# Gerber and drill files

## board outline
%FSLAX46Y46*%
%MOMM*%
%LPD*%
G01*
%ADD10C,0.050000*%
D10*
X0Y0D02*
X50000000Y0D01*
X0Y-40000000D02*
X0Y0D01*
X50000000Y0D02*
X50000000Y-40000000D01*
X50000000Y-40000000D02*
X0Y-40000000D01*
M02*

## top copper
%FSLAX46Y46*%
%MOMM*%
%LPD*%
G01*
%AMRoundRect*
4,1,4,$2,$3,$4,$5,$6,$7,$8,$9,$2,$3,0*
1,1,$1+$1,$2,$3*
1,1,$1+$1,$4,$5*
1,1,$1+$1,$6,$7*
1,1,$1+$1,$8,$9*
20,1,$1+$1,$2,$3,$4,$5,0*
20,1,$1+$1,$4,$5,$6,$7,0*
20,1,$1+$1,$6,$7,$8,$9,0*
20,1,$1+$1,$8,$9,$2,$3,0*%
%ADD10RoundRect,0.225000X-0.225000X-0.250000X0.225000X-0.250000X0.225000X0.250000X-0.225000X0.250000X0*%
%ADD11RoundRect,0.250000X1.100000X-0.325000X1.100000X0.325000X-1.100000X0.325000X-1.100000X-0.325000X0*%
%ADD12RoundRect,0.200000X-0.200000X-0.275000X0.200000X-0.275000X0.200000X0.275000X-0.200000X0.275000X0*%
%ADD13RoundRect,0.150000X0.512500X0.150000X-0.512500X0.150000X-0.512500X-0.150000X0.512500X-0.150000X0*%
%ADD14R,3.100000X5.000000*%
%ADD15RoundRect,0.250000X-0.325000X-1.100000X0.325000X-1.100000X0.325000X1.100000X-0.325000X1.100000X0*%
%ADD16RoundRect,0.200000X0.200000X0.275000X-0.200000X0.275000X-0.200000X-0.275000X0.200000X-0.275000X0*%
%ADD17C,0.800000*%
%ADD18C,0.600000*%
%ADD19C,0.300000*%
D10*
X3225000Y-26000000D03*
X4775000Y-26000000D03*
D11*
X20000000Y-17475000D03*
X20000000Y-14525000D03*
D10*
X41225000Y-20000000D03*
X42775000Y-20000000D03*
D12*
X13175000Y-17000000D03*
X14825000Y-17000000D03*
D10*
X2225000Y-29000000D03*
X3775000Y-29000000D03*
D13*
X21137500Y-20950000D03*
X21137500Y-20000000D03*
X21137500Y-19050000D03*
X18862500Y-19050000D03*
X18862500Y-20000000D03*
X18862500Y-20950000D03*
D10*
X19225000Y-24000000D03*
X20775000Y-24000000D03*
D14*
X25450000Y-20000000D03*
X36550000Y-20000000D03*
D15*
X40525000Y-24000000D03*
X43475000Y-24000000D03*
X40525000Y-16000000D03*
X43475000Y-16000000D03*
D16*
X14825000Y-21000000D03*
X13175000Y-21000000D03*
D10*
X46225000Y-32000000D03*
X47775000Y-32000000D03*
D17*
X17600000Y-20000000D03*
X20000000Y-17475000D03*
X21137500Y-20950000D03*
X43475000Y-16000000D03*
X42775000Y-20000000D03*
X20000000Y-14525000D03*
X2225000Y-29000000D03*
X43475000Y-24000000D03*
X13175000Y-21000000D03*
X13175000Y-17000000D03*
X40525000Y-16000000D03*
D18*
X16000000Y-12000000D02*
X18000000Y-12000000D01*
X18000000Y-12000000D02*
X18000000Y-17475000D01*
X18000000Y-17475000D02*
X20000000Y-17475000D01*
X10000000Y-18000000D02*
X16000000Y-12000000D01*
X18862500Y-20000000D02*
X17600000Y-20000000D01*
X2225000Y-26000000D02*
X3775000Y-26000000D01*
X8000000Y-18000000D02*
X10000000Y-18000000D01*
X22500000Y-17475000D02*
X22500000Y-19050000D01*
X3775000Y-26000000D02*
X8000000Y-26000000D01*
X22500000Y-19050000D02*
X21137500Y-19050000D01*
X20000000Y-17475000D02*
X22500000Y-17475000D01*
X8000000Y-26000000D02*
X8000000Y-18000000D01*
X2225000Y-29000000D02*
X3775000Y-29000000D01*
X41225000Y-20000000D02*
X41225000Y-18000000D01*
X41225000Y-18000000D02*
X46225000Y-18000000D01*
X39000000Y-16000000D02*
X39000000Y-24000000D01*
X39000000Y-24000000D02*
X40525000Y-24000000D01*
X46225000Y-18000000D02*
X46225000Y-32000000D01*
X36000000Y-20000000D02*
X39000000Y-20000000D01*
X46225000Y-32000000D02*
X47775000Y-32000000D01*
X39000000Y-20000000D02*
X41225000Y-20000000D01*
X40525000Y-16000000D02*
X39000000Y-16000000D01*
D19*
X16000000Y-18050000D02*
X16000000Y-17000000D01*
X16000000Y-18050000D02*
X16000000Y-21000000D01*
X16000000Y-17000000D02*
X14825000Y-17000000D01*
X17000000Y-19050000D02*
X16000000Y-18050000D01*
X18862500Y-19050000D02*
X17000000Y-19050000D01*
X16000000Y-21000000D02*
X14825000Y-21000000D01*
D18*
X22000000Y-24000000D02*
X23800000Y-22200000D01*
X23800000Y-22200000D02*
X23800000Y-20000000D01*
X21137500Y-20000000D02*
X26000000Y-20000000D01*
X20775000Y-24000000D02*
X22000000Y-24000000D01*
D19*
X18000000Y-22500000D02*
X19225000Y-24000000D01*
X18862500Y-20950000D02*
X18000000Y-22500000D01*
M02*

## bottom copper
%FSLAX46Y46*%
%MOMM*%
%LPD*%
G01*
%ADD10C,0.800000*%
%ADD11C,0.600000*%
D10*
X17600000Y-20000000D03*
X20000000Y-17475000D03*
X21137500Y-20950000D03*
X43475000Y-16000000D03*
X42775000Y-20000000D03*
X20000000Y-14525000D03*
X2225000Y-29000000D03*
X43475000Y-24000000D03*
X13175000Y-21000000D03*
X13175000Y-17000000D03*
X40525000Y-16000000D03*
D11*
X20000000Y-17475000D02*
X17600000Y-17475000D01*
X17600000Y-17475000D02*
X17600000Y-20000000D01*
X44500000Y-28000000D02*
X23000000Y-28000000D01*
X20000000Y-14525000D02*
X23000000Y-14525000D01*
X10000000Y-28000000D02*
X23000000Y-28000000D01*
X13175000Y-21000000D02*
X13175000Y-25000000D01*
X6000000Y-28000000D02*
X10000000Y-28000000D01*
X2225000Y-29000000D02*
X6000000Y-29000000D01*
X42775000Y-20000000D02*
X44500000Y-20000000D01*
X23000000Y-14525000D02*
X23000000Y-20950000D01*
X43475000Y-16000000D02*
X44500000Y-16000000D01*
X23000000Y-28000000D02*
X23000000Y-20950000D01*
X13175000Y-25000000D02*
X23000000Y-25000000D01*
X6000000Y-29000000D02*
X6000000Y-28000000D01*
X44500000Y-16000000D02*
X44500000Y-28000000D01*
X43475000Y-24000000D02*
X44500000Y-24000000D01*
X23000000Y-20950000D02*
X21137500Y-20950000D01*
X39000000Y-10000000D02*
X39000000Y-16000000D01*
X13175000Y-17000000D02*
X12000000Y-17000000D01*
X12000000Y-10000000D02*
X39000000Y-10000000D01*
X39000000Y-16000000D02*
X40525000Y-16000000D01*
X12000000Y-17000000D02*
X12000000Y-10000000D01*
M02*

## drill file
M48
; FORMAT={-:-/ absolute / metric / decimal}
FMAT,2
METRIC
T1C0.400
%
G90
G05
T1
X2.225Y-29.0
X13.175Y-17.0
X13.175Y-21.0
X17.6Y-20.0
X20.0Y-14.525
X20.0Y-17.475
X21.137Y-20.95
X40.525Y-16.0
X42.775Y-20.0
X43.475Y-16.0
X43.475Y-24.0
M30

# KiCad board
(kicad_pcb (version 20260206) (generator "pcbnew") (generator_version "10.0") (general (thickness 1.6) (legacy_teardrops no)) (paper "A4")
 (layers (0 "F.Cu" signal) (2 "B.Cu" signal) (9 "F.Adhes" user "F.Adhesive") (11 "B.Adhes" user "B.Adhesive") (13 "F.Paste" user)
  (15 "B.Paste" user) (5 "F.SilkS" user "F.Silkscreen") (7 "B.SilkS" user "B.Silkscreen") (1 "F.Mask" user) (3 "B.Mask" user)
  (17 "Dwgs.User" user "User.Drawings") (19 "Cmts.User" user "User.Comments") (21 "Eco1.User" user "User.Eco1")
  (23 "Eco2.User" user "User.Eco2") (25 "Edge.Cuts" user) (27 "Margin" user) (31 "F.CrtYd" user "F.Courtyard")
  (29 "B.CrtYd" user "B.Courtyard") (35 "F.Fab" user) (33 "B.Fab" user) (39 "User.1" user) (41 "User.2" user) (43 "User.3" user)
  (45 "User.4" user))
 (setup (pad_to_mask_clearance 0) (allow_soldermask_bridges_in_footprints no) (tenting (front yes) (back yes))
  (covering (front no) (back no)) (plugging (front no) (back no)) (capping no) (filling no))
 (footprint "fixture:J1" (layer "F.Cu") (at 4 26)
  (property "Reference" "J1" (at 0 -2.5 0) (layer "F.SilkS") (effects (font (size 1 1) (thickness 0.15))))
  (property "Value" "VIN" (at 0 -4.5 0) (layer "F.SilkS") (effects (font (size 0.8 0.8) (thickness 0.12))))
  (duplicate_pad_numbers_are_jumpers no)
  (pad "1" smd roundrect (at -0.775 0) (size 0.9 0.95) (layers "F.Cu" "F.Mask" "F.Paste") (roundrect_rratio 0.25) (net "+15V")
   (thermal_bridge_angle 45))
  (pad "2" smd roundrect (at 0.775 0) (size 0.9 0.95) (layers "F.Cu" "F.Mask" "F.Paste") (roundrect_rratio 0.25) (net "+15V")
   (thermal_bridge_angle 45)))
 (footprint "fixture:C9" (layer "F.Cu") (at 20 16 90)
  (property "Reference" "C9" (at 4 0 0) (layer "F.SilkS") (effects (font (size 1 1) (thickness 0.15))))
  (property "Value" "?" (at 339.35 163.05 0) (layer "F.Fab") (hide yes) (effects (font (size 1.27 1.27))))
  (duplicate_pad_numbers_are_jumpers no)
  (pad "1" smd roundrect (at -1.475 0 90) (size 1.15 2.7) (layers "F.Cu" "F.Mask" "F.Paste") (roundrect_rratio 0.217391) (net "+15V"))
  (pad "2" smd roundrect (at 1.475 0 90) (size 1.15 2.7) (layers "F.Cu" "F.Mask" "F.Paste") (roundrect_rratio 0.217391) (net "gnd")))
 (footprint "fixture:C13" (layer "F.Cu") (at 42 20)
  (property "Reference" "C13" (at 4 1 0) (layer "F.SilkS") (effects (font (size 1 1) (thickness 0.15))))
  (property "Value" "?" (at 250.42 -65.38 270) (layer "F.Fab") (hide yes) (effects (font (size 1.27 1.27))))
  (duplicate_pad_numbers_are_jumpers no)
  (pad "1" smd roundrect (at -0.775 0) (size 0.9 0.95) (layers "F.Cu" "F.Mask" "F.Paste") (roundrect_rratio 0.25) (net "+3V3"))
  (pad "2" smd roundrect (at 0.775 0) (size 0.9 0.95) (layers "F.Cu" "F.Mask" "F.Paste") (roundrect_rratio 0.25) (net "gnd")))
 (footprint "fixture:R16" (layer "F.Cu") (at 14 17)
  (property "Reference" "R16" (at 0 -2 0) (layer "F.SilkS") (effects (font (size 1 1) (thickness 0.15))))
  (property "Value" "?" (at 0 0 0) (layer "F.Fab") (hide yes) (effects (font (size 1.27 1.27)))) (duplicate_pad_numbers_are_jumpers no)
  (pad "1" smd roundrect (at -0.825 0) (size 0.8 0.95) (layers "F.Cu" "F.Mask" "F.Paste") (roundrect_rratio 0.25) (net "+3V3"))
  (pad "2" smd roundrect (at 0.825 0) (size 0.8 0.95) (layers "F.Cu" "F.Mask" "F.Paste") (roundrect_rratio 0.25) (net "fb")))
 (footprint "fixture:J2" (layer "F.Cu") (at 3 29)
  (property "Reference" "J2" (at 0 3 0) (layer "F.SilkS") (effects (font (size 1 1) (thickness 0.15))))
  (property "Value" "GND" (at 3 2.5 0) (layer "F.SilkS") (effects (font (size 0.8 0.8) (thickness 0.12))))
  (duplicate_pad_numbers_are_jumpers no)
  (pad "1" smd roundrect (at -0.775 0) (size 0.9 0.95) (layers "F.Cu" "F.Mask" "F.Paste") (roundrect_rratio 0.25) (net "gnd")
   (thermal_bridge_angle 45))
  (pad "2" smd roundrect (at 0.775 0) (size 0.9 0.95) (layers "F.Cu" "F.Mask" "F.Paste") (roundrect_rratio 0.25) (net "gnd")
   (thermal_bridge_angle 45)))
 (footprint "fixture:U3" (layer "F.Cu") (at 20 20 180)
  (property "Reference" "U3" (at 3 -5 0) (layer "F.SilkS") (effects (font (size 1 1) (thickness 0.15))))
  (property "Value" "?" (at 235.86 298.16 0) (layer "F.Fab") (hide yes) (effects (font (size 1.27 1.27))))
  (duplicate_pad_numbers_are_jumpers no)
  (pad "1" smd roundrect (at -1.1375 -0.95 180) (size 1.325 0.6) (layers "F.Cu" "F.Mask" "F.Paste") (roundrect_rratio 0.25) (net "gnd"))
  (pad "2" smd roundrect (at -1.1375 0 180) (size 1.325 0.6) (layers "F.Cu" "F.Mask" "F.Paste") (roundrect_rratio 0.25) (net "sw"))
  (pad "3" smd roundrect (at -1.1375 0.95 180) (size 1.325 0.6) (layers "F.Cu" "F.Mask" "F.Paste") (roundrect_rratio 0.25) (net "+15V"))
  (pad "4" smd roundrect (at 1.1375 0.95 180) (size 1.325 0.6) (layers "F.Cu" "F.Mask" "F.Paste") (roundrect_rratio 0.25) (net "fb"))
  (pad "5" smd roundrect (at 1.1375 0 180) (size 1.325 0.6) (layers "F.Cu" "F.Mask" "F.Paste") (roundrect_rratio 0.25) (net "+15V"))
  (pad "6" smd roundrect (at 1.1375 -0.95 180) (size 1.325 0.6) (layers "F.Cu" "F.Mask" "F.Paste") (roundrect_rratio 0.25) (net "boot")))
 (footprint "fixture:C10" (layer "F.Cu") (at 20 24)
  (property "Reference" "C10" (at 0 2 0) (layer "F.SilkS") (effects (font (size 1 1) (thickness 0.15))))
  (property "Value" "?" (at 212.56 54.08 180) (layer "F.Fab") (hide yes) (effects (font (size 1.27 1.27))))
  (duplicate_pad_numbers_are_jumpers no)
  (pad "1" smd roundrect (at -0.775 0) (size 0.9 0.95) (layers "F.Cu" "F.Mask" "F.Paste") (roundrect_rratio 0.25) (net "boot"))
  (pad "2" smd roundrect (at 0.775 0) (size 0.9 0.95) (layers "F.Cu" "F.Mask" "F.Paste") (roundrect_rratio 0.25) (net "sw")))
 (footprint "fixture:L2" (layer "F.Cu") (at 31 20)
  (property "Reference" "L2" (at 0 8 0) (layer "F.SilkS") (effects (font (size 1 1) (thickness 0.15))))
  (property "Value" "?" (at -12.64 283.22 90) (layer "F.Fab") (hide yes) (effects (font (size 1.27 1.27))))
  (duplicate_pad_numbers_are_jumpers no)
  (pad "1" smd rect (at -5.55 0) (size 3.1 5) (layers "F.Cu" "F.Mask" "F.Paste") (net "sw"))
  (pad "2" smd rect (at 5.55 0) (size 3.1 5) (layers "F.Cu" "F.Mask" "F.Paste") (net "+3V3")))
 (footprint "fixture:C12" (layer "F.Cu") (at 42 24)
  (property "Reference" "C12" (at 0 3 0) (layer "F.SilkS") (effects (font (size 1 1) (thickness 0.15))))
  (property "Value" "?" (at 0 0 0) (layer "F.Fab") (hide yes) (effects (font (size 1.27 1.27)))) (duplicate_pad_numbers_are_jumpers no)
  (pad "1" smd roundrect (at -1.475 0) (size 1.15 2.7) (layers "F.Cu" "F.Mask" "F.Paste") (roundrect_rratio 0.217391) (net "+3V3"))
  (pad "2" smd roundrect (at 1.475 0) (size 1.15 2.7) (layers "F.Cu" "F.Mask" "F.Paste") (roundrect_rratio 0.217391) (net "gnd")))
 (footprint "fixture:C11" (layer "F.Cu") (at 42 16)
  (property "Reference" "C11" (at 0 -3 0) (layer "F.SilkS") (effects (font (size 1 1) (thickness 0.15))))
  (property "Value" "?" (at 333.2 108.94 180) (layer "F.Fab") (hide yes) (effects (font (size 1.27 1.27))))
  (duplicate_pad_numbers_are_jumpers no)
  (pad "1" smd roundrect (at -1.475 0) (size 1.15 2.7) (layers "F.Cu" "F.Mask" "F.Paste") (roundrect_rratio 0.217391) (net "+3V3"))
  (pad "2" smd roundrect (at 1.475 0) (size 1.15 2.7) (layers "F.Cu" "F.Mask" "F.Paste") (roundrect_rratio 0.217391) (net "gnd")))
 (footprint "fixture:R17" (layer "F.Cu") (at 14 21 180)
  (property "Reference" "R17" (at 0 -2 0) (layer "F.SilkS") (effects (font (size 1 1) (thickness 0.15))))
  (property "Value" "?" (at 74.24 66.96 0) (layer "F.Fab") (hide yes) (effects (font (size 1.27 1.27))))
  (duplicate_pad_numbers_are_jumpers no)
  (pad "1" smd roundrect (at -0.825 0 180) (size 0.8 0.95) (layers "F.Cu" "F.Mask" "F.Paste") (roundrect_rratio 0.25) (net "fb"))
  (pad "2" smd roundrect (at 0.825 0 180) (size 0.8 0.95) (layers "F.Cu" "F.Mask" "F.Paste") (roundrect_rratio 0.25) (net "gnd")))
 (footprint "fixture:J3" (layer "F.Cu") (at 47 32)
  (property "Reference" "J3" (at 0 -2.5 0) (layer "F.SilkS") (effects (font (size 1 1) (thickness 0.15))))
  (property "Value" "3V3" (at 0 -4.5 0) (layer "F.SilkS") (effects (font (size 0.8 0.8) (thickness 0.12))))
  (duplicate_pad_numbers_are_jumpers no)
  (pad "1" smd roundrect (at -0.775 0) (size 0.9 0.95) (layers "F.Cu" "F.Mask" "F.Paste") (roundrect_rratio 0.25) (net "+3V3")
   (thermal_bridge_angle 45))
  (pad "2" smd roundrect (at 0.775 0) (size 0.9 0.95) (layers "F.Cu" "F.Mask" "F.Paste") (roundrect_rratio 0.25) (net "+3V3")
   (thermal_bridge_angle 45)))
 (gr_line (start 0 0) (end 50 0) (stroke (width 0.05) (type default)) (layer "Edge.Cuts"))
 (gr_line (start 0 40) (end 0 0) (stroke (width 0.05) (type default)) (layer "Edge.Cuts"))
 (gr_line (start 50 0) (end 50 40) (stroke (width 0.05) (type default)) (layer "Edge.Cuts"))
 (gr_line (start 50 40) (end 0 40) (stroke (width 0.05) (type default)) (layer "Edge.Cuts"))
 (segment (start 16 12) (end 18 12) (width 0.6) (layer "F.Cu") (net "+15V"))
 (segment (start 18 12) (end 18 17.475) (width 0.6) (layer "F.Cu") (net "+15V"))
 (segment (start 18 17.475) (end 20 17.475) (width 0.6) (layer "F.Cu") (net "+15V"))
 (segment (start 10 18) (end 16 12) (width 0.6) (layer "F.Cu") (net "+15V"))
 (segment (start 18.8625 20) (end 17.6 20) (width 0.6) (layer "F.Cu") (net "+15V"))
 (segment (start 2.225 26) (end 3.775 26) (width 0.6) (layer "F.Cu") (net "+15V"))
 (segment (start 8 18) (end 10 18) (width 0.6) (layer "F.Cu") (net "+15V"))
 (segment (start 22.5 17.475) (end 22.5 19.05) (width 0.6) (layer "F.Cu") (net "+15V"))
 (segment (start 3.775 26) (end 8 26) (width 0.6) (layer "F.Cu") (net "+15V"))
 (segment (start 22.5 19.05) (end 21.1375 19.05) (width 0.6) (layer "F.Cu") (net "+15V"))
 (segment (start 20 17.475) (end 22.5 17.475) (width 0.6) (layer "F.Cu") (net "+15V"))
 (segment (start 8 26) (end 8 18) (width 0.6) (layer "F.Cu") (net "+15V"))
 (via (at 17.6 20) (size 0.8) (drill 0.4) (layers "F.Cu" "B.Cu") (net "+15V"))
 (via (at 20 17.475) (size 0.8) (drill 0.4) (layers "F.Cu" "B.Cu") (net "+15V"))
 (segment (start 20 17.475) (end 17.6 17.475) (width 0.6) (layer "B.Cu") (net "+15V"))
 (segment (start 17.6 17.475) (end 17.6 20) (width 0.6) (layer "B.Cu") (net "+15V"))
 (segment (start 2.225 29) (end 3.775 29) (width 0.6) (layer "F.Cu") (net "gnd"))
 (via (at 21.1375 20.95) (size 0.8) (drill 0.4) (layers "F.Cu" "B.Cu") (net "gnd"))
 (via (at 43.475 16) (size 0.8) (drill 0.4) (layers "F.Cu" "B.Cu") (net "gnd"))
 (via (at 42.775 20) (size 0.8) (drill 0.4) (layers "F.Cu" "B.Cu") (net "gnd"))
 (via (at 20 14.525) (size 0.8) (drill 0.4) (layers "F.Cu" "B.Cu") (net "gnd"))
 (via (at 2.225 29) (size 0.8) (drill 0.4) (layers "F.Cu" "B.Cu") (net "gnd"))
 (via (at 43.475 24) (size 0.8) (drill 0.4) (layers "F.Cu" "B.Cu") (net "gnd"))
 (via (at 13.175 21) (size 0.8) (drill 0.4) (layers "F.Cu" "B.Cu") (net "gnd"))
 (segment (start 44.5 28) (end 23 28) (width 0.6) (layer "B.Cu") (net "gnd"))
 (segment (start 20 14.525) (end 23 14.525) (width 0.6) (layer "B.Cu") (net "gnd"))
 (segment (start 10 28) (end 23 28) (width 0.6) (layer "B.Cu") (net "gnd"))
 (segment (start 13.175 21) (end 13.175 25) (width 0.6) (layer "B.Cu") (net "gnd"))
 (segment (start 6 28) (end 10 28) (width 0.6) (layer "B.Cu") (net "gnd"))
 (segment (start 2.225 29) (end 6 29) (width 0.6) (layer "B.Cu") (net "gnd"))
 (segment (start 42.775 20) (end 44.5 20) (width 0.6) (layer "B.Cu") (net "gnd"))
 (segment (start 23 14.525) (end 23 20.95) (width 0.6) (layer "B.Cu") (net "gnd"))
 (segment (start 43.475 16) (end 44.5 16) (width 0.6) (layer "B.Cu") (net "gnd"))
 (segment (start 23 28) (end 23 20.95) (width 0.6) (layer "B.Cu") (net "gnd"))
 (segment (start 13.175 25) (end 23 25) (width 0.6) (layer "B.Cu") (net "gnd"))
 (segment (start 6 29) (end 6 28) (width 0.6) (layer "B.Cu") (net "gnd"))
 (segment (start 44.5 16) (end 44.5 28) (width 0.6) (layer "B.Cu") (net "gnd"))
 (segment (start 43.475 24) (end 44.5 24) (width 0.6) (layer "B.Cu") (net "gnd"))
 (segment (start 23 20.95) (end 21.1375 20.95) (width 0.6) (layer "B.Cu") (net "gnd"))
 (segment (start 41.225 20) (end 41.225 18) (width 0.6) (layer "F.Cu") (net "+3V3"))
 (segment (start 41.225 18) (end 46.225 18) (width 0.6) (layer "F.Cu") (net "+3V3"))
 (segment (start 39 16) (end 39 24) (width 0.6) (layer "F.Cu") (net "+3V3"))
 (segment (start 39 24) (end 40.525 24) (width 0.6) (layer "F.Cu") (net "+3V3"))
 (segment (start 46.225 18) (end 46.225 32) (width 0.6) (layer "F.Cu") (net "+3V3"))
 (segment (start 36 20) (end 39 20) (width 0.6) (layer "F.Cu") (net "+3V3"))
 (segment (start 46.225 32) (end 47.775 32) (width 0.6) (layer "F.Cu") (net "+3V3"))
 (segment (start 39 20) (end 41.225 20) (width 0.6) (layer "F.Cu") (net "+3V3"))
 (segment (start 40.525 16) (end 39 16) (width 0.6) (layer "F.Cu") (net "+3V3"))
 (via (at 13.175 17) (size 0.8) (drill 0.4) (layers "F.Cu" "B.Cu") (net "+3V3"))
 (via (at 40.525 16) (size 0.8) (drill 0.4) (layers "F.Cu" "B.Cu") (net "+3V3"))
 (segment (start 39 10) (end 39 16) (width 0.6) (layer "B.Cu") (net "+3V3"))
 (segment (start 13.175 17) (end 12 17) (width 0.6) (layer "B.Cu") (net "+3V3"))
 (segment (start 12 10) (end 39 10) (width 0.6) (layer "B.Cu") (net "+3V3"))
 (segment (start 39 16) (end 40.525 16) (width 0.6) (layer "B.Cu") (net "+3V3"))
 (segment (start 12 17) (end 12 10) (width 0.6) (layer "B.Cu") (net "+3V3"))
 (segment (start 16 18.05) (end 16 17) (width 0.3) (layer "F.Cu") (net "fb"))
 (segment (start 16 18.05) (end 16 21) (width 0.3) (layer "F.Cu") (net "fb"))
 (segment (start 16 17) (end 14.825 17) (width 0.3) (layer "F.Cu") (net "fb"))
 (segment (start 17 19.05) (end 16 18.05) (width 0.3) (layer "F.Cu") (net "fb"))
 (segment (start 18.8625 19.05) (end 17 19.05) (width 0.3) (layer "F.Cu") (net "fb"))
 (segment (start 16 21) (end 14.825 21) (width 0.3) (layer "F.Cu") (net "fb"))
 (segment (start 22 24) (end 23.8 22.2) (width 0.6) (layer "F.Cu") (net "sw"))
 (segment (start 23.8 22.2) (end 23.8 20) (width 0.6) (layer "F.Cu") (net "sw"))
 (segment (start 21.1375 20) (end 26 20) (width 0.6) (layer "F.Cu") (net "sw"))
 (segment (start 20.775 24) (end 22 24) (width 0.6) (layer "F.Cu") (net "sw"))
 (segment (start 18 22.5) (end 19.225 24) (width 0.3) (layer "F.Cu") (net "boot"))
 (segment (start 18.8625 20.95) (end 18 22.5) (width 0.3) (layer "F.Cu") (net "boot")))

